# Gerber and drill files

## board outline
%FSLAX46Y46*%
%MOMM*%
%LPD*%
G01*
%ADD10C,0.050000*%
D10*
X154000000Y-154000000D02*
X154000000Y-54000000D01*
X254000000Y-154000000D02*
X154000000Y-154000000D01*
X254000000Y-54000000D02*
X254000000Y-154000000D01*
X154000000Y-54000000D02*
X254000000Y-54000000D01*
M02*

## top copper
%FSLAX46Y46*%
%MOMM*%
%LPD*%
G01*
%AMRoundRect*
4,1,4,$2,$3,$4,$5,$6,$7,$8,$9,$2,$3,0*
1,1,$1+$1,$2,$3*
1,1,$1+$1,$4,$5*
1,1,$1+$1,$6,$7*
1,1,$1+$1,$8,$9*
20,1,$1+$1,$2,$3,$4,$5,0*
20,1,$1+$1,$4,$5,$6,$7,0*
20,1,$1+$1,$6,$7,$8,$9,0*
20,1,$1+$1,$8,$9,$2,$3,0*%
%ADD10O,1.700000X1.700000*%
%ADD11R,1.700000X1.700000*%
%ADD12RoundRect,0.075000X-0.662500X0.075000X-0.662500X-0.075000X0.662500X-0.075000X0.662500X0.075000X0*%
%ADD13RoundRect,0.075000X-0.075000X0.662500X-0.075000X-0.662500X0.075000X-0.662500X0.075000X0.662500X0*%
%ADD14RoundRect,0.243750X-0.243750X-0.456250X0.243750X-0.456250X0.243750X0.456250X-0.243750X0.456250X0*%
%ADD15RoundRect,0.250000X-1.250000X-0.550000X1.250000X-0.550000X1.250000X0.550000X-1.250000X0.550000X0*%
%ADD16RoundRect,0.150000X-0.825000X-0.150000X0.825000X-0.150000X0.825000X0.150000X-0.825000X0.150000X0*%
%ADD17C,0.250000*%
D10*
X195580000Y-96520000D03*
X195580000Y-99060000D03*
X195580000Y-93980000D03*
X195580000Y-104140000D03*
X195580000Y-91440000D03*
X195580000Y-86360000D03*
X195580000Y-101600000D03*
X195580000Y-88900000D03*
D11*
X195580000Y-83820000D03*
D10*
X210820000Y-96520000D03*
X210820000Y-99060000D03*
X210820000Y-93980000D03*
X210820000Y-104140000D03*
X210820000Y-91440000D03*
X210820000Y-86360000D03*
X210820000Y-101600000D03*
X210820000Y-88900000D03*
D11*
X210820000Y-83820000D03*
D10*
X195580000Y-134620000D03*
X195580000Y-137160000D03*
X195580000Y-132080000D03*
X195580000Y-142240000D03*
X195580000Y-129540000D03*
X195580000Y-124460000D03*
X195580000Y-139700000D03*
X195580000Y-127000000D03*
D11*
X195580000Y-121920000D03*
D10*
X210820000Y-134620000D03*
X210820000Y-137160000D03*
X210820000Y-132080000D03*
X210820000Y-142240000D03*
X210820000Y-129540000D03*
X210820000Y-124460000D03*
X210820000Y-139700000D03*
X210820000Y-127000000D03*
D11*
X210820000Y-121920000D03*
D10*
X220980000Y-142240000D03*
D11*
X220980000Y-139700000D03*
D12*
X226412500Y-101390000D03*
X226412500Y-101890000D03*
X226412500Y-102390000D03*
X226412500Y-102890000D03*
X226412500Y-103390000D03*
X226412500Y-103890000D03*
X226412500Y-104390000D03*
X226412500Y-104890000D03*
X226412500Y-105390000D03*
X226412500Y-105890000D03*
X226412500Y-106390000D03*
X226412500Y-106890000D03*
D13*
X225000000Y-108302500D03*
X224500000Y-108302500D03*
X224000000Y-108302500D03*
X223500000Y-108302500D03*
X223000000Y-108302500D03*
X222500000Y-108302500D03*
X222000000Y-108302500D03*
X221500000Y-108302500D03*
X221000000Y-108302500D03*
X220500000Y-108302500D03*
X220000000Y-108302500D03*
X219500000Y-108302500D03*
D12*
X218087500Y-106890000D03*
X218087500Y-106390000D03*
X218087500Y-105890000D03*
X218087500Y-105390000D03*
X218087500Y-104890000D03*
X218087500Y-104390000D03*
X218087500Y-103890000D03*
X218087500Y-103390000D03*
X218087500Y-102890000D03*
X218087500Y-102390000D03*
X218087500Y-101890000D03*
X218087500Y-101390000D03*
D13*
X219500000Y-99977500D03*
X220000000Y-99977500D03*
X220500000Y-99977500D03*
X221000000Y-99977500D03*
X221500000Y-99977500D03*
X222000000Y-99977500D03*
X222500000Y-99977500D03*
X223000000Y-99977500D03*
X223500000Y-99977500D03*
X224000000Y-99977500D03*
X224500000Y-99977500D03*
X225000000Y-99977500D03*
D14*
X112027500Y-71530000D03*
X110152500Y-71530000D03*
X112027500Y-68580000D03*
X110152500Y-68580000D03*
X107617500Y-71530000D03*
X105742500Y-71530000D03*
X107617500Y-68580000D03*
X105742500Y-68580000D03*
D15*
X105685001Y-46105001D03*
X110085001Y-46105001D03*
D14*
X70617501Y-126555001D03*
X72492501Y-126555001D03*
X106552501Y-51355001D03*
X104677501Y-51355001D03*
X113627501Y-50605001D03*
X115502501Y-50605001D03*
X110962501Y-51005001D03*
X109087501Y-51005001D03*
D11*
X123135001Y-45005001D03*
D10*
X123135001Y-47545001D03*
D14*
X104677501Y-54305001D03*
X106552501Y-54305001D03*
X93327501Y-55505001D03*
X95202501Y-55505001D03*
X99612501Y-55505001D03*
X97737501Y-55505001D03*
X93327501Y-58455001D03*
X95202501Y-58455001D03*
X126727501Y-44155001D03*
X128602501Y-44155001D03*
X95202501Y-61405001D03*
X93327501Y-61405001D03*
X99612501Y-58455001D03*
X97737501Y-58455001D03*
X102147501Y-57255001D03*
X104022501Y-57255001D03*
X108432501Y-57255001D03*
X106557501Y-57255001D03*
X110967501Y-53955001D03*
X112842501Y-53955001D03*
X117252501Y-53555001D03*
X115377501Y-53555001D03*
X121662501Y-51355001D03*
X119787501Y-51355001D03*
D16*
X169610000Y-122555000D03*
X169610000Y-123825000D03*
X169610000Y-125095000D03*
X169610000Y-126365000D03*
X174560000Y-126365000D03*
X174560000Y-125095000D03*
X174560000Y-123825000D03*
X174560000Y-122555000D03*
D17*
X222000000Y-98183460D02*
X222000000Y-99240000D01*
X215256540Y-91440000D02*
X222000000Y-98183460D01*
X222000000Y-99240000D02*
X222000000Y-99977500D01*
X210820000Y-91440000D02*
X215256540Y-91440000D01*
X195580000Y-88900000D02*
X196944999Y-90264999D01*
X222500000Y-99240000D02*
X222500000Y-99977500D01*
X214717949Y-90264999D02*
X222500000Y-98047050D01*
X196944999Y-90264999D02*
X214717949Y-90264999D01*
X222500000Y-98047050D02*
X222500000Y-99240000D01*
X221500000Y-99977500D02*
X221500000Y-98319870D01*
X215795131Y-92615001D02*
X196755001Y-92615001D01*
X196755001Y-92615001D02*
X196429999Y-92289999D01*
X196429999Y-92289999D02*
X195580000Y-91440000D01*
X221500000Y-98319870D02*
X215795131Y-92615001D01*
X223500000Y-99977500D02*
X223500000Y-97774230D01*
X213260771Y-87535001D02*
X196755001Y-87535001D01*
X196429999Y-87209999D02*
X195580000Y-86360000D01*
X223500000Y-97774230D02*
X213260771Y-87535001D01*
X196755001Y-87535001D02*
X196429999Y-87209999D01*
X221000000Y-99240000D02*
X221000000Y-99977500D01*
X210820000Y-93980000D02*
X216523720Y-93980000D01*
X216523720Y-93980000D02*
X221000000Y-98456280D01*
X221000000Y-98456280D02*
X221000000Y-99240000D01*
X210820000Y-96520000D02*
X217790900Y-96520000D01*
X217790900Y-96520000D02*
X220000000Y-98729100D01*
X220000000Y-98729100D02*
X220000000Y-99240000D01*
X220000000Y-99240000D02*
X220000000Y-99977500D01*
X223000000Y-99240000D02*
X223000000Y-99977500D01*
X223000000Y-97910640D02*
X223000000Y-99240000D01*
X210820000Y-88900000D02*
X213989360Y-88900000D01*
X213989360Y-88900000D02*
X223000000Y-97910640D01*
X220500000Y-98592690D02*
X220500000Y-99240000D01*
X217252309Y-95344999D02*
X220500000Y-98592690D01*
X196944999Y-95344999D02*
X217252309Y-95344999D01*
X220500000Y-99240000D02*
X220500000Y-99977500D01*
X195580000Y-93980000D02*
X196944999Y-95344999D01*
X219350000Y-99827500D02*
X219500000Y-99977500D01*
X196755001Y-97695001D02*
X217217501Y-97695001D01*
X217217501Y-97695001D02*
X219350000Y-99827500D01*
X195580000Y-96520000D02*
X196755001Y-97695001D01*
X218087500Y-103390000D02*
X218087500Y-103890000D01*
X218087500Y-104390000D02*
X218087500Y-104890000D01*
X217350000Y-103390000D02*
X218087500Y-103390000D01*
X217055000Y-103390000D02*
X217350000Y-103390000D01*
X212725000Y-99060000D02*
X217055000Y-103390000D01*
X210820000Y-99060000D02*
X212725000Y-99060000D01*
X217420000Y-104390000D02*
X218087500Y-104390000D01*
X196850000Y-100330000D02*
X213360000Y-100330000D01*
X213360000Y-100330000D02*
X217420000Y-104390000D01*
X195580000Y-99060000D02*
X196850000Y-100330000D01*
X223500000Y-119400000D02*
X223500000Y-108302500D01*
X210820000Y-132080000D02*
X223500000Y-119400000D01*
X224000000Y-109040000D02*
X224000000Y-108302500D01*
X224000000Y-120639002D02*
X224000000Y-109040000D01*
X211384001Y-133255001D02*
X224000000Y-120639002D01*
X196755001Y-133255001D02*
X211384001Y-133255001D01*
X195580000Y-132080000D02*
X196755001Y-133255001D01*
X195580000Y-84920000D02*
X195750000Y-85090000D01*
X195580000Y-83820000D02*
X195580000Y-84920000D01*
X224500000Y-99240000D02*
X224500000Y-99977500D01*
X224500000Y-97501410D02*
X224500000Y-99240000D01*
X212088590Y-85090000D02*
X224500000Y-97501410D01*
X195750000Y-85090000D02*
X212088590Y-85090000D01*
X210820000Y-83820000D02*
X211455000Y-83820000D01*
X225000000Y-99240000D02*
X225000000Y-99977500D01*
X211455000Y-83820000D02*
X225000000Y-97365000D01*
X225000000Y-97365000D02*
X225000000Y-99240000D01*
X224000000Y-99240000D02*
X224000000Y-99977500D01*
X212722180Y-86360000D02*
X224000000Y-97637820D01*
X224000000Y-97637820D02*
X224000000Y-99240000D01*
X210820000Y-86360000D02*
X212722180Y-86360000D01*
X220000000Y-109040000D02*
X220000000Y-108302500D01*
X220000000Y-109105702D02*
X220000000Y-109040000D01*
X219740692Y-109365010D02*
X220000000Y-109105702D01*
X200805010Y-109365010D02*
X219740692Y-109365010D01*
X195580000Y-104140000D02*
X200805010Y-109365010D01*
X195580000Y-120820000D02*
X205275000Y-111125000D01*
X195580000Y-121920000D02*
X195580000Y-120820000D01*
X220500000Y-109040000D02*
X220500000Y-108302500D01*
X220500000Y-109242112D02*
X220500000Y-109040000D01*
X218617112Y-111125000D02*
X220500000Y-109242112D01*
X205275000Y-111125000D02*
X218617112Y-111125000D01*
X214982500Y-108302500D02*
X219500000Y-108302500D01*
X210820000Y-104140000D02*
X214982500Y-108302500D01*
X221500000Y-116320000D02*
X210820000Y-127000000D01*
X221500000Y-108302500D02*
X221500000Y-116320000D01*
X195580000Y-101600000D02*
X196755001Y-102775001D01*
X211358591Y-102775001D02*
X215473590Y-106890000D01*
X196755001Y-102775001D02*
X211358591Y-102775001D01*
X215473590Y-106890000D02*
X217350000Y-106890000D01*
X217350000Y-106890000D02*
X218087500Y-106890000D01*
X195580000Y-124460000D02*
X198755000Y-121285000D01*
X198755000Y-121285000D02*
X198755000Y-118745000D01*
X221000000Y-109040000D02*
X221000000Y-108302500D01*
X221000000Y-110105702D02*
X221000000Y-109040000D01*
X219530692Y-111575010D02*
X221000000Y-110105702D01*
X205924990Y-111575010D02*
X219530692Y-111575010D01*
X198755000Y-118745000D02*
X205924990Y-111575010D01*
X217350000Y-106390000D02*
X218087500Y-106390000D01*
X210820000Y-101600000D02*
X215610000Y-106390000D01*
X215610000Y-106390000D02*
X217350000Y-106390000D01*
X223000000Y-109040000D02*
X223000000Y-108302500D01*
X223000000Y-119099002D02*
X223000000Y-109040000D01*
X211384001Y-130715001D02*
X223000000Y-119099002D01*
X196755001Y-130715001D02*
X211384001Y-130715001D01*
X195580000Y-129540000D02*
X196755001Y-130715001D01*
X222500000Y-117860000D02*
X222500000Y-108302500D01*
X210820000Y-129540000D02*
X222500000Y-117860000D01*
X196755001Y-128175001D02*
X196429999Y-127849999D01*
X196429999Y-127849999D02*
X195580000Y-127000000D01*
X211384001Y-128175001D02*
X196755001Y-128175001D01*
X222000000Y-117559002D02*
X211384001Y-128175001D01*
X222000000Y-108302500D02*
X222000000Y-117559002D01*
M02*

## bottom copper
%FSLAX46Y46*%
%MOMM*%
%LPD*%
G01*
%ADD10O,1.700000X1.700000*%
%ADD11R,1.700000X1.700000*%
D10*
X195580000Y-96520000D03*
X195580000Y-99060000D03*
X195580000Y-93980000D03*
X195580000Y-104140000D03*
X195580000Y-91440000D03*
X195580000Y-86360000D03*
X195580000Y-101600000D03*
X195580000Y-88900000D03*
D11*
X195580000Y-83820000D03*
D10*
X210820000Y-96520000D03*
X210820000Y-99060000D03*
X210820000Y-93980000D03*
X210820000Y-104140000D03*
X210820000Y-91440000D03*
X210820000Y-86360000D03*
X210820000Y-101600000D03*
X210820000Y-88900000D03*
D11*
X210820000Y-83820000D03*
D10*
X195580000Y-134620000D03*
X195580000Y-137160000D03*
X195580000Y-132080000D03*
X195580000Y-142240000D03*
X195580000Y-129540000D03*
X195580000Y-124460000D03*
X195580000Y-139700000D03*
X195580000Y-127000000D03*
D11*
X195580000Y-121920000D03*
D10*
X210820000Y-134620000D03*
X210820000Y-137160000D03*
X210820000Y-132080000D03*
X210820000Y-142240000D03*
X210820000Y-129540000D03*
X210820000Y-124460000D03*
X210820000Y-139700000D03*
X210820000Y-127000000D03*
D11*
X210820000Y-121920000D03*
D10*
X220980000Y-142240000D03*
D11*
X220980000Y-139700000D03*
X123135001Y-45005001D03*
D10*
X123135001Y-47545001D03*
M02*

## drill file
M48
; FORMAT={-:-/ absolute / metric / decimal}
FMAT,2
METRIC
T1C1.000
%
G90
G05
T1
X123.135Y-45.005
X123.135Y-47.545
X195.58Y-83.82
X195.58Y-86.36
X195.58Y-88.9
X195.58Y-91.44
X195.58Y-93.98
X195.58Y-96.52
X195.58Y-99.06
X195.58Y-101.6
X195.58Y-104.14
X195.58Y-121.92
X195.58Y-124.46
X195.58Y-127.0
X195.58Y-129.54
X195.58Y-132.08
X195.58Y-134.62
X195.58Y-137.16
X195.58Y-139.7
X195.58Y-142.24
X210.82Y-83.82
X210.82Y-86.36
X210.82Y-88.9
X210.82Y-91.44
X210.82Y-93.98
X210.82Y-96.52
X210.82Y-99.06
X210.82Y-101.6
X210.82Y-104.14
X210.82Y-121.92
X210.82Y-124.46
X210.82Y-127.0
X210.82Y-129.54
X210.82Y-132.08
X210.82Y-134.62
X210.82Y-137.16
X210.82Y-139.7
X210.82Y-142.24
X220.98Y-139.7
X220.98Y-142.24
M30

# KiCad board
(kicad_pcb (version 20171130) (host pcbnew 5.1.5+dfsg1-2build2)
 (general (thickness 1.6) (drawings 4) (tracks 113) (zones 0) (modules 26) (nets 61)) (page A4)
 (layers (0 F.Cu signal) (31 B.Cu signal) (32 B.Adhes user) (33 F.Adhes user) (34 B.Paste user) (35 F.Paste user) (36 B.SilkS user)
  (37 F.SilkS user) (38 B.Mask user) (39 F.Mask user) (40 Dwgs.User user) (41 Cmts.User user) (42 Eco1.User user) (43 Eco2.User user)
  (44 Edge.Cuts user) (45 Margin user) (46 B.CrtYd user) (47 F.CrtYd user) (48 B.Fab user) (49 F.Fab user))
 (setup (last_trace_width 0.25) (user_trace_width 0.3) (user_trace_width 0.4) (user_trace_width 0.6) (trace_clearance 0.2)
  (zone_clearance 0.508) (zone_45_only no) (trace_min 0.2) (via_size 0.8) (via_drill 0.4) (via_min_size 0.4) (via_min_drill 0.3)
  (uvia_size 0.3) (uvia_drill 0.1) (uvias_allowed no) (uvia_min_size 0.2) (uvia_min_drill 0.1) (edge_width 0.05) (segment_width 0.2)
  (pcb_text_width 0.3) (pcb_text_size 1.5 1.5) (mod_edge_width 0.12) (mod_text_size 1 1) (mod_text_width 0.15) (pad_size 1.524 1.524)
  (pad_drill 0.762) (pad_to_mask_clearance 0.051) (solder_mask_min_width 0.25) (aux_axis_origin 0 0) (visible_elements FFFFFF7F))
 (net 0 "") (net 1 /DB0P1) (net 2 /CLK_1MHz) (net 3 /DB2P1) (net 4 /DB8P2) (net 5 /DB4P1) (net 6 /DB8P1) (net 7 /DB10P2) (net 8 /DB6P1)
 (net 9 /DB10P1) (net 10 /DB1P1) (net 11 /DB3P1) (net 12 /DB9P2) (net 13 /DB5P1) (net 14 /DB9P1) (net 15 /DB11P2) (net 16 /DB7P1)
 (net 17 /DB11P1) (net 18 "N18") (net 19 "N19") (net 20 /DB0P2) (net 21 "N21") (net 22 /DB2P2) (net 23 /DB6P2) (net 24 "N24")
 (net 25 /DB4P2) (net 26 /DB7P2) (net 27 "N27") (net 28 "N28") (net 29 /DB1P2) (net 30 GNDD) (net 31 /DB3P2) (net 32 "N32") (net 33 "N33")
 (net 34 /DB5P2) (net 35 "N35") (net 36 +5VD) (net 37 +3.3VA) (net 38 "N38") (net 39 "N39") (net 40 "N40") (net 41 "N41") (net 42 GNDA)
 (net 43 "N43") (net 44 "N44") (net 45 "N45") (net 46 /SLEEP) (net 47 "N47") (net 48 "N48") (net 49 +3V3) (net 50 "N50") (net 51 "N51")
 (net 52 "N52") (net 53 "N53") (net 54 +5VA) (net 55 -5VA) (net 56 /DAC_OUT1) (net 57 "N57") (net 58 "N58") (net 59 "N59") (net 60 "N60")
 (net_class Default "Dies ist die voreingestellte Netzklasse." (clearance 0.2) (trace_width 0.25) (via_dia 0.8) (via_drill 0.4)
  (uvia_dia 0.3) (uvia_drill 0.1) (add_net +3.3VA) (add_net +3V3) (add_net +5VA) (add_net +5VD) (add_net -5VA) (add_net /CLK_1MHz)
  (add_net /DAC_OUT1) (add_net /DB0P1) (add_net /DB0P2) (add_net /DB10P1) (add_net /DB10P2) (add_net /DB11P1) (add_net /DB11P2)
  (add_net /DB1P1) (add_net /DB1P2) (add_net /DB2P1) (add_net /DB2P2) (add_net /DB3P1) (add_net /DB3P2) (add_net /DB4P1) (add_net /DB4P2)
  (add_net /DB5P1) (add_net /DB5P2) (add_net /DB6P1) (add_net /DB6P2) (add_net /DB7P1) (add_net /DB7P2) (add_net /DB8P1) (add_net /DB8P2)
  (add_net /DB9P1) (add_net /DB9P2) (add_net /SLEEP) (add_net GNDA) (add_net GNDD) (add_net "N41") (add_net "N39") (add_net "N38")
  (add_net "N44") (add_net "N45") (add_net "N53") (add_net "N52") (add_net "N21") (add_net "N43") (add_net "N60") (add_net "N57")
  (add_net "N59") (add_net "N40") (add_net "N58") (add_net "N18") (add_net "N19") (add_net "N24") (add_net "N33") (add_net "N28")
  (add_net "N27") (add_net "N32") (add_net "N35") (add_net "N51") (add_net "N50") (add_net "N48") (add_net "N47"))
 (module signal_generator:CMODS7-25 (layer F.Cu) (at 195.58 83.82)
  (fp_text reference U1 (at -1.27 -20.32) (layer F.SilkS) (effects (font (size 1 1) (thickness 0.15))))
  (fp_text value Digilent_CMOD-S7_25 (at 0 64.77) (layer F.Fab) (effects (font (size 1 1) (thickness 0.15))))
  (pad 6 thru_hole oval (at 0 12.7) (size 1.7 1.7) (drill 1) (layers *.Cu *.Mask) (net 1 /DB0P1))
  (pad 7 thru_hole oval (at 0 15.24) (size 1.7 1.7) (drill 1) (layers *.Cu *.Mask) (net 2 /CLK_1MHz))
  (pad 5 thru_hole oval (at 0 10.16) (size 1.7 1.7) (drill 1) (layers *.Cu *.Mask) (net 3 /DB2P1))
  (pad 9 thru_hole oval (at 0 20.32) (size 1.7 1.7) (drill 1) (layers *.Cu *.Mask) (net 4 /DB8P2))
  (pad 4 thru_hole oval (at 0 7.62) (size 1.7 1.7) (drill 1) (layers *.Cu *.Mask) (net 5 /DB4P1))
  (pad 2 thru_hole oval (at 0 2.54) (size 1.7 1.7) (drill 1) (layers *.Cu *.Mask) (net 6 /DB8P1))
  (pad 8 thru_hole oval (at 0 17.78) (size 1.7 1.7) (drill 1) (layers *.Cu *.Mask) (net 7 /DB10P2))
  (pad 3 thru_hole oval (at 0 5.08) (size 1.7 1.7) (drill 1) (layers *.Cu *.Mask) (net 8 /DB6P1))
  (pad 1 thru_hole rect (at 0 0) (size 1.7 1.7) (drill 1) (layers *.Cu *.Mask) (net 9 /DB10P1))
  (pad 43 thru_hole oval (at 15.24 12.7) (size 1.7 1.7) (drill 1) (layers *.Cu *.Mask) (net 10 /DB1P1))
  (pad 42 thru_hole oval (at 15.24 15.24) (size 1.7 1.7) (drill 1) (layers *.Cu *.Mask) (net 2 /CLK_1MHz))
  (pad 44 thru_hole oval (at 15.24 10.16) (size 1.7 1.7) (drill 1) (layers *.Cu *.Mask) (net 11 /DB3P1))
  (pad 40 thru_hole oval (at 15.24 20.32) (size 1.7 1.7) (drill 1) (layers *.Cu *.Mask) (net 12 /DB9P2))
  (pad 45 thru_hole oval (at 15.24 7.62) (size 1.7 1.7) (drill 1) (layers *.Cu *.Mask) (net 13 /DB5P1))
  (pad 47 thru_hole oval (at 15.24 2.54) (size 1.7 1.7) (drill 1) (layers *.Cu *.Mask) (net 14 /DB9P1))
  (pad 41 thru_hole oval (at 15.24 17.78) (size 1.7 1.7) (drill 1) (layers *.Cu *.Mask) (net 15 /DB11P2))
  (pad 46 thru_hole oval (at 15.24 5.08) (size 1.7 1.7) (drill 1) (layers *.Cu *.Mask) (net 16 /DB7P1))
  (pad 48 thru_hole rect (at 15.24 0) (size 1.7 1.7) (drill 1) (layers *.Cu *.Mask) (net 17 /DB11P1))
  (pad 21 thru_hole oval (at 0 50.8) (size 1.7 1.7) (drill 1) (layers *.Cu *.Mask) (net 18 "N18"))
  (pad 22 thru_hole oval (at 0 53.34) (size 1.7 1.7) (drill 1) (layers *.Cu *.Mask) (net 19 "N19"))
  (pad 20 thru_hole oval (at 0 48.26) (size 1.7 1.7) (drill 1) (layers *.Cu *.Mask) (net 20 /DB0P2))
  (pad 24 thru_hole oval (at 0 58.42) (size 1.7 1.7) (drill 1) (layers *.Cu *.Mask) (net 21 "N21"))
  (pad 19 thru_hole oval (at 0 45.72) (size 1.7 1.7) (drill 1) (layers *.Cu *.Mask) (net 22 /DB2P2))
  (pad 17 thru_hole oval (at 0 40.64) (size 1.7 1.7) (drill 1) (layers *.Cu *.Mask) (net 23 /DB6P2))
  (pad 23 thru_hole oval (at 0 55.88) (size 1.7 1.7) (drill 1) (layers *.Cu *.Mask) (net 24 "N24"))
  (pad 18 thru_hole oval (at 0 43.18) (size 1.7 1.7) (drill 1) (layers *.Cu *.Mask) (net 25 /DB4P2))
  (pad 16 thru_hole rect (at 0 38.1) (size 1.7 1.7) (drill 1) (layers *.Cu *.Mask) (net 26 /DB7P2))
  (pad 28 thru_hole oval (at 15.24 50.8) (size 1.7 1.7) (drill 1) (layers *.Cu *.Mask) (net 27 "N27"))
  (pad 27 thru_hole oval (at 15.24 53.34) (size 1.7 1.7) (drill 1) (layers *.Cu *.Mask) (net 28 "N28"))
  (pad 29 thru_hole oval (at 15.24 48.26) (size 1.7 1.7) (drill 1) (layers *.Cu *.Mask) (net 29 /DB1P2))
  (pad 25 thru_hole oval (at 15.24 58.42) (size 1.7 1.7) (drill 1) (layers *.Cu *.Mask) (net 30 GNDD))
  (pad 30 thru_hole oval (at 15.24 45.72) (size 1.7 1.7) (drill 1) (layers *.Cu *.Mask) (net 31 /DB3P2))
  (pad 32 thru_hole oval (at 15.24 40.64) (size 1.7 1.7) (drill 1) (layers *.Cu *.Mask) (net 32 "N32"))
  (pad 26 thru_hole oval (at 15.24 55.88) (size 1.7 1.7) (drill 1) (layers *.Cu *.Mask) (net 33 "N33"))
  (pad 31 thru_hole oval (at 15.24 43.18) (size 1.7 1.7) (drill 1) (layers *.Cu *.Mask) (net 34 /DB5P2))
  (pad 33 thru_hole rect (at 15.24 38.1) (size 1.7 1.7) (drill 1) (layers *.Cu *.Mask) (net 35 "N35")))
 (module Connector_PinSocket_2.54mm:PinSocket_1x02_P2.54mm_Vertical (layer F.Cu) (at 220.98 139.7)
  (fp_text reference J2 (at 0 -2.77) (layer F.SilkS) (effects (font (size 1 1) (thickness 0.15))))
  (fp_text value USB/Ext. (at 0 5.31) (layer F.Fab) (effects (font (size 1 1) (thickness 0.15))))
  (pad 2 thru_hole oval (at 0 2.54) (size 1.7 1.7) (drill 1) (layers *.Cu *.Mask) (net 21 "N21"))
  (pad 1 thru_hole rect (at 0 0) (size 1.7 1.7) (drill 1) (layers *.Cu *.Mask) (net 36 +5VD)))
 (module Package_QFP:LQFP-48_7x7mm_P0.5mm (layer F.Cu) (at 222.25 104.14 270)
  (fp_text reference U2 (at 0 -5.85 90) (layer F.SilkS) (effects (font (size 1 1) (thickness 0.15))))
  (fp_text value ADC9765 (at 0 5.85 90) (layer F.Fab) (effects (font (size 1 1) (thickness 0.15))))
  (pad 48 smd roundrect (at -2.75 -4.1625 270) (size 0.3 1.475) (layers F.Cu F.Paste F.Mask) (roundrect_rratio 0.25) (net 36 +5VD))
  (pad 47 smd roundrect (at -2.25 -4.1625 270) (size 0.3 1.475) (layers F.Cu F.Paste F.Mask) (roundrect_rratio 0.25) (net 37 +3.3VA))
  (pad 46 smd roundrect (at -1.75 -4.1625 270) (size 0.3 1.475) (layers F.Cu F.Paste F.Mask) (roundrect_rratio 0.25) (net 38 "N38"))
  (pad 45 smd roundrect (at -1.25 -4.1625 270) (size 0.3 1.475) (layers F.Cu F.Paste F.Mask) (roundrect_rratio 0.25) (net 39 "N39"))
  (pad 44 smd roundrect (at -0.75 -4.1625 270) (size 0.3 1.475) (layers F.Cu F.Paste F.Mask) (roundrect_rratio 0.25) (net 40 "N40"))
  (pad 43 smd roundrect (at -0.25 -4.1625 270) (size 0.3 1.475) (layers F.Cu F.Paste F.Mask) (roundrect_rratio 0.25) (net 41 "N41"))
  (pad 42 smd roundrect (at 0.25 -4.1625 270) (size 0.3 1.475) (layers F.Cu F.Paste F.Mask) (roundrect_rratio 0.25) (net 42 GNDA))
  (pad 41 smd roundrect (at 0.75 -4.1625 270) (size 0.3 1.475) (layers F.Cu F.Paste F.Mask) (roundrect_rratio 0.25) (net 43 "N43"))
  (pad 40 smd roundrect (at 1.25 -4.1625 270) (size 0.3 1.475) (layers F.Cu F.Paste F.Mask) (roundrect_rratio 0.25) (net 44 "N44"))
  (pad 39 smd roundrect (at 1.75 -4.1625 270) (size 0.3 1.475) (layers F.Cu F.Paste F.Mask) (roundrect_rratio 0.25) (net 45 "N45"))
  (pad 38 smd roundrect (at 2.25 -4.1625 270) (size 0.3 1.475) (layers F.Cu F.Paste F.Mask) (roundrect_rratio 0.25) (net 42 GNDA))
  (pad 37 smd roundrect (at 2.75 -4.1625 270) (size 0.3 1.475) (layers F.Cu F.Paste F.Mask) (roundrect_rratio 0.25) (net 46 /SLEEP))
  (pad 36 smd roundrect (at 4.1625 -2.75 270) (size 1.475 0.3) (layers F.Cu F.Paste F.Mask) (roundrect_rratio 0.25) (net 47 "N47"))
  (pad 35 smd roundrect (at 4.1625 -2.25 270) (size 1.475 0.3) (layers F.Cu F.Paste F.Mask) (roundrect_rratio 0.25) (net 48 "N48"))
  (pad 34 smd roundrect (at 4.1625 -1.75 270) (size 1.475 0.3) (layers F.Cu F.Paste F.Mask) (roundrect_rratio 0.25) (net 20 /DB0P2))
  (pad 33 smd roundrect (at 4.1625 -1.25 270) (size 1.475 0.3) (layers F.Cu F.Paste F.Mask) (roundrect_rratio 0.25) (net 29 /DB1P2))
  (pad 32 smd roundrect (at 4.1625 -0.75 270) (size 1.475 0.3) (layers F.Cu F.Paste F.Mask) (roundrect_rratio 0.25) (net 22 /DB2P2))
  (pad 31 smd roundrect (at 4.1625 -0.25 270) (size 1.475 0.3) (layers F.Cu F.Paste F.Mask) (roundrect_rratio 0.25) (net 31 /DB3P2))
  (pad 30 smd roundrect (at 4.1625 0.25 270) (size 1.475 0.3) (layers F.Cu F.Paste F.Mask) (roundrect_rratio 0.25) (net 25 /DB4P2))
  (pad 29 smd roundrect (at 4.1625 0.75 270) (size 1.475 0.3) (layers F.Cu F.Paste F.Mask) (roundrect_rratio 0.25) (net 34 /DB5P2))
  (pad 28 smd roundrect (at 4.1625 1.25 270) (size 1.475 0.3) (layers F.Cu F.Paste F.Mask) (roundrect_rratio 0.25) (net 23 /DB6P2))
  (pad 27 smd roundrect (at 4.1625 1.75 270) (size 1.475 0.3) (layers F.Cu F.Paste F.Mask) (roundrect_rratio 0.25) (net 26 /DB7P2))
  (pad 26 smd roundrect (at 4.1625 2.25 270) (size 1.475 0.3) (layers F.Cu F.Paste F.Mask) (roundrect_rratio 0.25) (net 4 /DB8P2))
  (pad 25 smd roundrect (at 4.1625 2.75 270) (size 1.475 0.3) (layers F.Cu F.Paste F.Mask) (roundrect_rratio 0.25) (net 12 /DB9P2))
  (pad 24 smd roundrect (at 2.75 4.1625 270) (size 0.3 1.475) (layers F.Cu F.Paste F.Mask) (roundrect_rratio 0.25) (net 7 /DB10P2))
  (pad 23 smd roundrect (at 2.25 4.1625 270) (size 0.3 1.475) (layers F.Cu F.Paste F.Mask) (roundrect_rratio 0.25) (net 15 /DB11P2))
  (pad 22 smd roundrect (at 1.75 4.1625 270) (size 0.3 1.475) (layers F.Cu F.Paste F.Mask) (roundrect_rratio 0.25) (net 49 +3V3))
  (pad 21 smd roundrect (at 1.25 4.1625 270) (size 0.3 1.475) (layers F.Cu F.Paste F.Mask) (roundrect_rratio 0.25) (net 30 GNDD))
  (pad 20 smd roundrect (at 0.75 4.1625 270) (size 0.3 1.475) (layers F.Cu F.Paste F.Mask) (roundrect_rratio 0.25) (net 2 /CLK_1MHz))
  (pad 19 smd roundrect (at 0.25 4.1625 270) (size 0.3 1.475) (layers F.Cu F.Paste F.Mask) (roundrect_rratio 0.25) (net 2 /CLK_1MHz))
  (pad 18 smd roundrect (at -0.25 4.1625 270) (size 0.3 1.475) (layers F.Cu F.Paste F.Mask) (roundrect_rratio 0.25) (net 2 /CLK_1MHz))
  (pad 17 smd roundrect (at -0.75 4.1625 270) (size 0.3 1.475) (layers F.Cu F.Paste F.Mask) (roundrect_rratio 0.25) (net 2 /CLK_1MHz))
  (pad 16 smd roundrect (at -1.25 4.1625 270) (size 0.3 1.475) (layers F.Cu F.Paste F.Mask) (roundrect_rratio 0.25) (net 49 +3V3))
  (pad 15 smd roundrect (at -1.75 4.1625 270) (size 0.3 1.475) (layers F.Cu F.Paste F.Mask) (roundrect_rratio 0.25) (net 30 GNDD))
  (pad 14 smd roundrect (at -2.25 4.1625 270) (size 0.3 1.475) (layers F.Cu F.Paste F.Mask) (roundrect_rratio 0.25) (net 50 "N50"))
  (pad 13 smd roundrect (at -2.75 4.1625 270) (size 0.3 1.475) (layers F.Cu F.Paste F.Mask) (roundrect_rratio 0.25) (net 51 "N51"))
  (pad 12 smd roundrect (at -4.1625 2.75 270) (size 1.475 0.3) (layers F.Cu F.Paste F.Mask) (roundrect_rratio 0.25) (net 1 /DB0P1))
  (pad 11 smd roundrect (at -4.1625 2.25 270) (size 1.475 0.3) (layers F.Cu F.Paste F.Mask) (roundrect_rratio 0.25) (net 10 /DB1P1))
  (pad 10 smd roundrect (at -4.1625 1.75 270) (size 1.475 0.3) (layers F.Cu F.Paste F.Mask) (roundrect_rratio 0.25) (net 3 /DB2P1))
  (pad 9 smd roundrect (at -4.1625 1.25 270) (size 1.475 0.3) (layers F.Cu F.Paste F.Mask) (roundrect_rratio 0.25) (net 11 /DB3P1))
  (pad 8 smd roundrect (at -4.1625 0.75 270) (size 1.475 0.3) (layers F.Cu F.Paste F.Mask) (roundrect_rratio 0.25) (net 5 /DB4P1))
  (pad 7 smd roundrect (at -4.1625 0.25 270) (size 1.475 0.3) (layers F.Cu F.Paste F.Mask) (roundrect_rratio 0.25) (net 13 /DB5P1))
  (pad 6 smd roundrect (at -4.1625 -0.25 270) (size 1.475 0.3) (layers F.Cu F.Paste F.Mask) (roundrect_rratio 0.25) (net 8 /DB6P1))
  (pad 5 smd roundrect (at -4.1625 -0.75 270) (size 1.475 0.3) (layers F.Cu F.Paste F.Mask) (roundrect_rratio 0.25) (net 16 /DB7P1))
  (pad 4 smd roundrect (at -4.1625 -1.25 270) (size 1.475 0.3) (layers F.Cu F.Paste F.Mask) (roundrect_rratio 0.25) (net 6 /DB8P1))
  (pad 3 smd roundrect (at -4.1625 -1.75 270) (size 1.475 0.3) (layers F.Cu F.Paste F.Mask) (roundrect_rratio 0.25) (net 14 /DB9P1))
  (pad 2 smd roundrect (at -4.1625 -2.25 270) (size 1.475 0.3) (layers F.Cu F.Paste F.Mask) (roundrect_rratio 0.25) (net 9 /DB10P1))
  (pad 1 smd roundrect (at -4.1625 -2.75 270) (size 1.475 0.3) (layers F.Cu F.Paste F.Mask) (roundrect_rratio 0.25) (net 17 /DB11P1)))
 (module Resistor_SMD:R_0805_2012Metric (layer F.Cu) (at 111.09 71.53)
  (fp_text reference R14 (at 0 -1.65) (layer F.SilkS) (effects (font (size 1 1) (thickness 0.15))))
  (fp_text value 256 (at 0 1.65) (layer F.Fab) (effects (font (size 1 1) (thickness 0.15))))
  (pad 2 smd roundrect (at 0.9375 0) (size 0.975 1.4) (layers F.Cu F.Paste F.Mask) (roundrect_rratio 0.25) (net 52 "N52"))
  (pad 1 smd roundrect (at -0.9375 0) (size 0.975 1.4) (layers F.Cu F.Paste F.Mask) (roundrect_rratio 0.25) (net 40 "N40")))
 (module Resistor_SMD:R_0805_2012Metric (layer F.Cu) (at 111.09 68.58)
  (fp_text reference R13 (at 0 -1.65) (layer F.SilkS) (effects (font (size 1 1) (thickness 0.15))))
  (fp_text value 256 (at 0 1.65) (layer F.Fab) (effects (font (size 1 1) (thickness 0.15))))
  (pad 2 smd roundrect (at 0.9375 0) (size 0.975 1.4) (layers F.Cu F.Paste F.Mask) (roundrect_rratio 0.25) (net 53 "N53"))
  (pad 1 smd roundrect (at -0.9375 0) (size 0.975 1.4) (layers F.Cu F.Paste F.Mask) (roundrect_rratio 0.25) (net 43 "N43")))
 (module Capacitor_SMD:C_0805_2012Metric (layer F.Cu) (at 106.68 71.53)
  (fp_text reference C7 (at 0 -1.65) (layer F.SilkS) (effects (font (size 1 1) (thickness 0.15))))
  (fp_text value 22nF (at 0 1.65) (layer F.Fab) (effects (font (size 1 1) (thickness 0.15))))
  (pad 2 smd roundrect (at 0.9375 0) (size 0.975 1.4) (layers F.Cu F.Paste F.Mask) (roundrect_rratio 0.25) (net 42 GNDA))
  (pad 1 smd roundrect (at -0.9375 0) (size 0.975 1.4) (layers F.Cu F.Paste F.Mask) (roundrect_rratio 0.25) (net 52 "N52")))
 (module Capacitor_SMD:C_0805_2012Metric (layer F.Cu) (at 106.68 68.58)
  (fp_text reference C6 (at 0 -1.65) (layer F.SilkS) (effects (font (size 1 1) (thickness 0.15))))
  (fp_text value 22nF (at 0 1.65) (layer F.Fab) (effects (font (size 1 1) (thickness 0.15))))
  (pad 2 smd roundrect (at 0.9375 0) (size 0.975 1.4) (layers F.Cu F.Paste F.Mask) (roundrect_rratio 0.25) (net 42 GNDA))
  (pad 1 smd roundrect (at -0.9375 0) (size 0.975 1.4) (layers F.Cu F.Paste F.Mask) (roundrect_rratio 0.25) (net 53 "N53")))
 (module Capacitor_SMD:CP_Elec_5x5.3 (layer F.Cu) (at 107.885001 46.105001)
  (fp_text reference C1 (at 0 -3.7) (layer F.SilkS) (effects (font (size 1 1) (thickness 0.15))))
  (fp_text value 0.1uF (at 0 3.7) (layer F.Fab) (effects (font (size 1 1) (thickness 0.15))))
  (pad 1 smd roundrect (at -2.2 0) (size 3 1.6) (layers F.Cu F.Paste F.Mask) (roundrect_rratio 0.15625) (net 41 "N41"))
  (pad 2 smd roundrect (at 2.2 0) (size 3 1.6) (layers F.Cu F.Paste F.Mask) (roundrect_rratio 0.15625) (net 42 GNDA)))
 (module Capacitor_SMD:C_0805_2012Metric (layer F.Cu) (at 71.555001 126.555001)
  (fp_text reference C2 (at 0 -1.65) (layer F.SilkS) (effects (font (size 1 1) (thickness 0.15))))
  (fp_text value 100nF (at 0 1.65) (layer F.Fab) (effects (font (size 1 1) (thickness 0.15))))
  (pad 1 smd roundrect (at -0.9375 0) (size 0.975 1.4) (layers F.Cu F.Paste F.Mask) (roundrect_rratio 0.25) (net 39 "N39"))
  (pad 2 smd roundrect (at 0.9375 0) (size 0.975 1.4) (layers F.Cu F.Paste F.Mask) (roundrect_rratio 0.25) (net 38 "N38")))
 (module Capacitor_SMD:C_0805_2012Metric (layer F.Cu) (at 105.615001 51.355001)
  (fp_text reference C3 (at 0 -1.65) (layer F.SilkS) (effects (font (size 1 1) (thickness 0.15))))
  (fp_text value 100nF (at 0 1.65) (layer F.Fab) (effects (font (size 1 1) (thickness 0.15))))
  (pad 2 smd roundrect (at 0.9375 0) (size 0.975 1.4) (layers F.Cu F.Paste F.Mask) (roundrect_rratio 0.25) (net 45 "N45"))
  (pad 1 smd roundrect (at -0.9375 0) (size 0.975 1.4) (layers F.Cu F.Paste F.Mask) (roundrect_rratio 0.25) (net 44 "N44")))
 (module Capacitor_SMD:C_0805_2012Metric (layer F.Cu) (at 114.565001 50.605001)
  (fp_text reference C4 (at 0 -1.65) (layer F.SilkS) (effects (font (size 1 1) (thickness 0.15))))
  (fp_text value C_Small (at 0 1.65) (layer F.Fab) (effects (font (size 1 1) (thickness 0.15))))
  (pad 1 smd roundrect (at -0.9375 0) (size 0.975 1.4) (layers F.Cu F.Paste F.Mask) (roundrect_rratio 0.25) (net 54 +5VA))
  (pad 2 smd roundrect (at 0.9375 0) (size 0.975 1.4) (layers F.Cu F.Paste F.Mask) (roundrect_rratio 0.25) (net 42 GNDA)))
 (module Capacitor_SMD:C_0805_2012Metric (layer F.Cu) (at 110.025001 51.005001)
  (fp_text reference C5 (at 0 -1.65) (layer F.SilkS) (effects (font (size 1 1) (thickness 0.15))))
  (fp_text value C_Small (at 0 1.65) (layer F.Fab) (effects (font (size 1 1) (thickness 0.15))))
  (pad 2 smd roundrect (at 0.9375 0) (size 0.975 1.4) (layers F.Cu F.Paste F.Mask) (roundrect_rratio 0.25) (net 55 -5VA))
  (pad 1 smd roundrect (at -0.9375 0) (size 0.975 1.4) (layers F.Cu F.Paste F.Mask) (roundrect_rratio 0.25) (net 42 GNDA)))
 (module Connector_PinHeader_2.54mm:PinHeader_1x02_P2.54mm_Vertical (layer F.Cu) (at 123.135001 45.005001)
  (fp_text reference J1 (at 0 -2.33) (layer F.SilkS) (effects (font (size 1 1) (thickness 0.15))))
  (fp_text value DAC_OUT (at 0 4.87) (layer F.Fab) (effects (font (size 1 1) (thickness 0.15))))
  (pad 1 thru_hole rect (at 0 0) (size 1.7 1.7) (drill 1) (layers *.Cu *.Mask) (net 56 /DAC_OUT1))
  (pad 2 thru_hole oval (at 0 2.54) (size 1.7 1.7) (drill 1) (layers *.Cu *.Mask) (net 56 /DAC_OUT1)))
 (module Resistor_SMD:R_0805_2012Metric (layer F.Cu) (at 105.615001 54.305001)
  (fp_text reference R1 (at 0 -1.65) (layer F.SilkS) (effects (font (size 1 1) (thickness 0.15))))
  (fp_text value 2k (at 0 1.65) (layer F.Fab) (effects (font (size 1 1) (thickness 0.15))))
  (pad 1 smd roundrect (at -0.9375 0) (size 0.975 1.4) (layers F.Cu F.Paste F.Mask) (roundrect_rratio 0.25) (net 43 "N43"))
  (pad 2 smd roundrect (at 0.9375 0) (size 0.975 1.4) (layers F.Cu F.Paste F.Mask) (roundrect_rratio 0.25) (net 42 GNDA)))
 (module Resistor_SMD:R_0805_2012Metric (layer F.Cu) (at 94.265001 55.505001)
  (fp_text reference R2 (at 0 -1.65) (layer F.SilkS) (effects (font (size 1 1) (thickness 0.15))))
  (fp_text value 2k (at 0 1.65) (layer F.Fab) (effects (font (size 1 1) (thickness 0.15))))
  (pad 1 smd roundrect (at -0.9375 0) (size 0.975 1.4) (layers F.Cu F.Paste F.Mask) (roundrect_rratio 0.25) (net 40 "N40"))
  (pad 2 smd roundrect (at 0.9375 0) (size 0.975 1.4) (layers F.Cu F.Paste F.Mask) (roundrect_rratio 0.25) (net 42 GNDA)))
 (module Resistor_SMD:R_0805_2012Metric (layer F.Cu) (at 98.675001 55.505001)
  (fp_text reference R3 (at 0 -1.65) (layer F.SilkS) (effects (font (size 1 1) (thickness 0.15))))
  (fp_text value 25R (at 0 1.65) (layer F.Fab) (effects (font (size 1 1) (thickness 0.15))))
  (pad 2 smd roundrect (at 0.9375 0) (size 0.975 1.4) (layers F.Cu F.Paste F.Mask) (roundrect_rratio 0.25) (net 42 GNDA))
  (pad 1 smd roundrect (at -0.9375 0) (size 0.975 1.4) (layers F.Cu F.Paste F.Mask) (roundrect_rratio 0.25) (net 39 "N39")))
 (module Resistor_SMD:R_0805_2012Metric (layer F.Cu) (at 94.265001 58.455001)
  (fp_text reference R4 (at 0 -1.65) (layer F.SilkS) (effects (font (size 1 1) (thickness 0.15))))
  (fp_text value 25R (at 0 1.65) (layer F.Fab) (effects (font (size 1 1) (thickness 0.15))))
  (pad 1 smd roundrect (at -0.9375 0) (size 0.975 1.4) (layers F.Cu F.Paste F.Mask) (roundrect_rratio 0.25) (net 44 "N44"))
  (pad 2 smd roundrect (at 0.9375 0) (size 0.975 1.4) (layers F.Cu F.Paste F.Mask) (roundrect_rratio 0.25) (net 42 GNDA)))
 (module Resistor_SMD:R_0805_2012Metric (layer F.Cu) (at 127.665001 44.155001)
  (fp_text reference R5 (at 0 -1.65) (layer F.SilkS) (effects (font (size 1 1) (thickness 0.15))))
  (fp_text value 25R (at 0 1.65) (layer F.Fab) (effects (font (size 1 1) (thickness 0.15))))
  (pad 1 smd roundrect (at -0.9375 0) (size 0.975 1.4) (layers F.Cu F.Paste F.Mask) (roundrect_rratio 0.25) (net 38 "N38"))
  (pad 2 smd roundrect (at 0.9375 0) (size 0.975 1.4) (layers F.Cu F.Paste F.Mask) (roundrect_rratio 0.25) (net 42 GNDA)))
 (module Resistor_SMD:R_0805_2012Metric (layer F.Cu) (at 94.265001 61.405001)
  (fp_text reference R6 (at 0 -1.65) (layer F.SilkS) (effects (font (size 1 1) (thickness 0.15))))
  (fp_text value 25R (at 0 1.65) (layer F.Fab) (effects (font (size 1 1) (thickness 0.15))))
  (pad 2 smd roundrect (at 0.9375 0) (size 0.975 1.4) (layers F.Cu F.Paste F.Mask) (roundrect_rratio 0.25) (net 42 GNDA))
  (pad 1 smd roundrect (at -0.9375 0) (size 0.975 1.4) (layers F.Cu F.Paste F.Mask) (roundrect_rratio 0.25) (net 45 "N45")))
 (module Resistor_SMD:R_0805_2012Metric (layer F.Cu) (at 98.675001 58.455001)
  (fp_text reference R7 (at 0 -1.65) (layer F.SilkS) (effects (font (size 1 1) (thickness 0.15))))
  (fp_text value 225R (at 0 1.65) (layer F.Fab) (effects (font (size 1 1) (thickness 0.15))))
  (pad 2 smd roundrect (at 0.9375 0) (size 0.975 1.4) (layers F.Cu F.Paste F.Mask) (roundrect_rratio 0.25) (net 38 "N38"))
  (pad 1 smd roundrect (at -0.9375 0) (size 0.975 1.4) (layers F.Cu F.Paste F.Mask) (roundrect_rratio 0.25) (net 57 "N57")))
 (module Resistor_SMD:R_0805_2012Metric (layer F.Cu) (at 103.085001 57.255001)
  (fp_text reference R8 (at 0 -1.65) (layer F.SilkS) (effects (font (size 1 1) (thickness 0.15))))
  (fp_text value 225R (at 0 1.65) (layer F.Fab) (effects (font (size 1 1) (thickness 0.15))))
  (pad 1 smd roundrect (at -0.9375 0) (size 0.975 1.4) (layers F.Cu F.Paste F.Mask) (roundrect_rratio 0.25) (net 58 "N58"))
  (pad 2 smd roundrect (at 0.9375 0) (size 0.975 1.4) (layers F.Cu F.Paste F.Mask) (roundrect_rratio 0.25) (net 39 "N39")))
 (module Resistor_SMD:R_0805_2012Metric (layer F.Cu) (at 107.495001 57.255001)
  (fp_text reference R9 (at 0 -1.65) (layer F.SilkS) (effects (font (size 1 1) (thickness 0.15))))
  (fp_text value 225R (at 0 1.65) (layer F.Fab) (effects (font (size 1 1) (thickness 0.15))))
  (pad 2 smd roundrect (at 0.9375 0) (size 0.975 1.4) (layers F.Cu F.Paste F.Mask) (roundrect_rratio 0.25) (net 45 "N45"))
  (pad 1 smd roundrect (at -0.9375 0) (size 0.975 1.4) (layers F.Cu F.Paste F.Mask) (roundrect_rratio 0.25) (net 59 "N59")))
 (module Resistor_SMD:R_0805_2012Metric (layer F.Cu) (at 111.905001 53.955001)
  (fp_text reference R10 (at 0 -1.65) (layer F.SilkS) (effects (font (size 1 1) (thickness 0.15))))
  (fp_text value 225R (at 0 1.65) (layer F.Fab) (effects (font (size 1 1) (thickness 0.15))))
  (pad 1 smd roundrect (at -0.9375 0) (size 0.975 1.4) (layers F.Cu F.Paste F.Mask) (roundrect_rratio 0.25) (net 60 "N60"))
  (pad 2 smd roundrect (at 0.9375 0) (size 0.975 1.4) (layers F.Cu F.Paste F.Mask) (roundrect_rratio 0.25) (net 44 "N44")))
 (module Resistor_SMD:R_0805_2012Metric (layer F.Cu) (at 116.315001 53.555001)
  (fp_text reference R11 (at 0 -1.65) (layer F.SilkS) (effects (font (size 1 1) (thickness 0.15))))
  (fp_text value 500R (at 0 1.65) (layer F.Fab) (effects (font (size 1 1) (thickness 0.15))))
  (pad 2 smd roundrect (at 0.9375 0) (size 0.975 1.4) (layers F.Cu F.Paste F.Mask) (roundrect_rratio 0.25) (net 57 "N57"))
  (pad 1 smd roundrect (at -0.9375 0) (size 0.975 1.4) (layers F.Cu F.Paste F.Mask) (roundrect_rratio 0.25) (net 56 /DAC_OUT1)))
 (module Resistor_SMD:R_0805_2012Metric (layer F.Cu) (at 120.725001 51.355001)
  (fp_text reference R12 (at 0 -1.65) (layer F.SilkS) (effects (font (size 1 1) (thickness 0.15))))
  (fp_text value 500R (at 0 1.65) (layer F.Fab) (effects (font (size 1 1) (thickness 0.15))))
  (pad 2 smd roundrect (at 0.9375 0) (size 0.975 1.4) (layers F.Cu F.Paste F.Mask) (roundrect_rratio 0.25) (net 59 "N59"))
  (pad 1 smd roundrect (at -0.9375 0) (size 0.975 1.4) (layers F.Cu F.Paste F.Mask) (roundrect_rratio 0.25) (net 56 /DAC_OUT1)))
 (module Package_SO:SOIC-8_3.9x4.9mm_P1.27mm (layer F.Cu) (at 172.085 124.46)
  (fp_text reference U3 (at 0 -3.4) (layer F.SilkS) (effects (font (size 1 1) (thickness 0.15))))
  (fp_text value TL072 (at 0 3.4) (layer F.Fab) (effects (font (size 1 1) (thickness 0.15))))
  (pad 1 smd roundrect (at -2.475 -1.905) (size 1.95 0.6) (layers F.Cu F.Paste F.Mask) (roundrect_rratio 0.25) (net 56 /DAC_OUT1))
  (pad 2 smd roundrect (at -2.475 -0.635) (size 1.95 0.6) (layers F.Cu F.Paste F.Mask) (roundrect_rratio 0.25) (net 57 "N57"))
  (pad 3 smd roundrect (at -2.475 0.635) (size 1.95 0.6) (layers F.Cu F.Paste F.Mask) (roundrect_rratio 0.25) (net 58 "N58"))
  (pad 4 smd roundrect (at -2.475 1.905) (size 1.95 0.6) (layers F.Cu F.Paste F.Mask) (roundrect_rratio 0.25) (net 55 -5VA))
  (pad 5 smd roundrect (at 2.475 1.905) (size 1.95 0.6) (layers F.Cu F.Paste F.Mask) (roundrect_rratio 0.25) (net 60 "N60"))
  (pad 6 smd roundrect (at 2.475 0.635) (size 1.95 0.6) (layers F.Cu F.Paste F.Mask) (roundrect_rratio 0.25) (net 59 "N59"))
  (pad 7 smd roundrect (at 2.475 -0.635) (size 1.95 0.6) (layers F.Cu F.Paste F.Mask) (roundrect_rratio 0.25) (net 56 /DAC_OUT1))
  (pad 8 smd roundrect (at 2.475 -1.905) (size 1.95 0.6) (layers F.Cu F.Paste F.Mask) (roundrect_rratio 0.25) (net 54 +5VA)))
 (gr_line (start 154 154) (end 154 54) (layer Edge.Cuts) (width 0.05))
 (gr_line (start 254 154) (end 154 154) (layer Edge.Cuts) (width 0.05))
 (gr_line (start 254 54) (end 254 154) (layer Edge.Cuts) (width 0.05))
 (gr_line (start 154 54) (end 254 54) (layer Edge.Cuts) (width 0.05))
 (segment (start 222 98.18346) (end 222 99.24) (width 0.25) (layer F.Cu) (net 13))
 (segment (start 215.25654 91.44) (end 222 98.18346) (width 0.25) (layer F.Cu) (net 13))
 (segment (start 222 99.24) (end 222 99.9775) (width 0.25) (layer F.Cu) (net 13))
 (segment (start 210.82 91.44) (end 215.25654 91.44) (width 0.25) (layer F.Cu) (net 13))
 (segment (start 195.58 88.9) (end 196.944999 90.264999) (width 0.25) (layer F.Cu) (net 8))
 (segment (start 222.5 99.24) (end 222.5 99.9775) (width 0.25) (layer F.Cu) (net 8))
 (segment (start 214.717949 90.264999) (end 222.5 98.04705) (width 0.25) (layer F.Cu) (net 8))
 (segment (start 196.944999 90.264999) (end 214.717949 90.264999) (width 0.25) (layer F.Cu) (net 8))
 (segment (start 222.5 98.04705) (end 222.5 99.24) (width 0.25) (layer F.Cu) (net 8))
 (segment (start 221.5 99.9775) (end 221.5 98.31987) (width 0.25) (layer F.Cu) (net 5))
 (segment (start 215.795131 92.615001) (end 196.755001 92.615001) (width 0.25) (layer F.Cu) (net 5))
 (segment (start 196.755001 92.615001) (end 196.429999 92.289999) (width 0.25) (layer F.Cu) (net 5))
 (segment (start 196.429999 92.289999) (end 195.58 91.44) (width 0.25) (layer F.Cu) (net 5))
 (segment (start 221.5 98.31987) (end 215.795131 92.615001) (width 0.25) (layer F.Cu) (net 5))
 (segment (start 223.5 99.9775) (end 223.5 97.77423) (width 0.25) (layer F.Cu) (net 6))
 (segment (start 213.260771 87.535001) (end 196.755001 87.535001) (width 0.25) (layer F.Cu) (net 6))
 (segment (start 196.429999 87.209999) (end 195.58 86.36) (width 0.25) (layer F.Cu) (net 6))
 (segment (start 223.5 97.77423) (end 213.260771 87.535001) (width 0.25) (layer F.Cu) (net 6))
 (segment (start 196.755001 87.535001) (end 196.429999 87.209999) (width 0.25) (layer F.Cu) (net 6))
 (segment (start 221 99.24) (end 221 99.9775) (width 0.25) (layer F.Cu) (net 11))
 (segment (start 210.82 93.98) (end 216.52372 93.98) (width 0.25) (layer F.Cu) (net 11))
 (segment (start 216.52372 93.98) (end 221 98.45628) (width 0.25) (layer F.Cu) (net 11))
 (segment (start 221 98.45628) (end 221 99.24) (width 0.25) (layer F.Cu) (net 11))
 (segment (start 210.82 96.52) (end 217.7909 96.52) (width 0.25) (layer F.Cu) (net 10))
 (segment (start 217.7909 96.52) (end 220 98.7291) (width 0.25) (layer F.Cu) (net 10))
 (segment (start 220 98.7291) (end 220 99.24) (width 0.25) (layer F.Cu) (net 10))
 (segment (start 220 99.24) (end 220 99.9775) (width 0.25) (layer F.Cu) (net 10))
 (segment (start 223 99.24) (end 223 99.9775) (width 0.25) (layer F.Cu) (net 16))
 (segment (start 223 97.91064) (end 223 99.24) (width 0.25) (layer F.Cu) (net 16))
 (segment (start 210.82 88.9) (end 213.98936 88.9) (width 0.25) (layer F.Cu) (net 16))
 (segment (start 213.98936 88.9) (end 223 97.91064) (width 0.25) (layer F.Cu) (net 16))
 (segment (start 220.5 98.59269) (end 220.5 99.24) (width 0.25) (layer F.Cu) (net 3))
 (segment (start 217.252309 95.344999) (end 220.5 98.59269) (width 0.25) (layer F.Cu) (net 3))
 (segment (start 196.944999 95.344999) (end 217.252309 95.344999) (width 0.25) (layer F.Cu) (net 3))
 (segment (start 220.5 99.24) (end 220.5 99.9775) (width 0.25) (layer F.Cu) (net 3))
 (segment (start 195.58 93.98) (end 196.944999 95.344999) (width 0.25) (layer F.Cu) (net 3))
 (segment (start 219.35 99.8275) (end 219.5 99.9775) (width 0.25) (layer F.Cu) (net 1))
 (segment (start 196.755001 97.695001) (end 217.217501 97.695001) (width 0.25) (layer F.Cu) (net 1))
 (segment (start 217.217501 97.695001) (end 219.35 99.8275) (width 0.25) (layer F.Cu) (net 1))
 (segment (start 195.58 96.52) (end 196.755001 97.695001) (width 0.25) (layer F.Cu) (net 1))
 (segment (start 218.0875 103.39) (end 218.0875 103.89) (width 0.25) (layer F.Cu) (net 2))
 (segment (start 218.0875 104.39) (end 218.0875 104.89) (width 0.25) (layer F.Cu) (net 2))
 (segment (start 217.35 103.39) (end 218.0875 103.39) (width 0.25) (layer F.Cu) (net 2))
 (segment (start 217.055 103.39) (end 217.35 103.39) (width 0.25) (layer F.Cu) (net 2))
 (segment (start 212.725 99.06) (end 217.055 103.39) (width 0.25) (layer F.Cu) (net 2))
 (segment (start 210.82 99.06) (end 212.725 99.06) (width 0.25) (layer F.Cu) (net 2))
 (segment (start 217.42 104.39) (end 218.0875 104.39) (width 0.25) (layer F.Cu) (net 2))
 (segment (start 196.85 100.33) (end 213.36 100.33) (width 0.25) (layer F.Cu) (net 2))
 (segment (start 213.36 100.33) (end 217.42 104.39) (width 0.25) (layer F.Cu) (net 2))
 (segment (start 195.58 99.06) (end 196.85 100.33) (width 0.25) (layer F.Cu) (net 2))
 (segment (start 223.5 119.4) (end 223.5 108.3025) (width 0.25) (layer F.Cu) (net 29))
 (segment (start 210.82 132.08) (end 223.5 119.4) (width 0.25) (layer F.Cu) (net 29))
 (segment (start 224 109.04) (end 224 108.3025) (width 0.25) (layer F.Cu) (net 20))
 (segment (start 224 120.639002) (end 224 109.04) (width 0.25) (layer F.Cu) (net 20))
 (segment (start 211.384001 133.255001) (end 224 120.639002) (width 0.25) (layer F.Cu) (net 20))
 (segment (start 196.755001 133.255001) (end 211.384001 133.255001) (width 0.25) (layer F.Cu) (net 20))
 (segment (start 195.58 132.08) (end 196.755001 133.255001) (width 0.25) (layer F.Cu) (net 20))
 (segment (start 195.58 84.92) (end 195.75 85.09) (width 0.25) (layer F.Cu) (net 9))
 (segment (start 195.58 83.82) (end 195.58 84.92) (width 0.25) (layer F.Cu) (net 9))
 (segment (start 224.5 99.24) (end 224.5 99.9775) (width 0.25) (layer F.Cu) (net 9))
 (segment (start 224.5 97.50141) (end 224.5 99.24) (width 0.25) (layer F.Cu) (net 9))
 (segment (start 212.08859 85.09) (end 224.5 97.50141) (width 0.25) (layer F.Cu) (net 9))
 (segment (start 195.75 85.09) (end 212.08859 85.09) (width 0.25) (layer F.Cu) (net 9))
 (segment (start 210.82 83.82) (end 211.455 83.82) (width 0.25) (layer F.Cu) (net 17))
 (segment (start 225 99.24) (end 225 99.9775) (width 0.25) (layer F.Cu) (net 17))
 (segment (start 211.455 83.82) (end 225 97.365) (width 0.25) (layer F.Cu) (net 17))
 (segment (start 225 97.365) (end 225 99.24) (width 0.25) (layer F.Cu) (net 17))
 (segment (start 224 99.24) (end 224 99.9775) (width 0.25) (layer F.Cu) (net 14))
 (segment (start 212.72218 86.36) (end 224 97.63782) (width 0.25) (layer F.Cu) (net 14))
 (segment (start 224 97.63782) (end 224 99.24) (width 0.25) (layer F.Cu) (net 14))
 (segment (start 210.82 86.36) (end 212.72218 86.36) (width 0.25) (layer F.Cu) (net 14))
 (segment (start 220 109.04) (end 220 108.3025) (width 0.25) (layer F.Cu) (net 4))
 (segment (start 220 109.105702) (end 220 109.04) (width 0.25) (layer F.Cu) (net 4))
 (segment (start 219.740692 109.36501) (end 220 109.105702) (width 0.25) (layer F.Cu) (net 4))
 (segment (start 200.80501 109.36501) (end 219.740692 109.36501) (width 0.25) (layer F.Cu) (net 4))
 (segment (start 195.58 104.14) (end 200.80501 109.36501) (width 0.25) (layer F.Cu) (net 4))
 (segment (start 195.58 120.82) (end 205.275 111.125) (width 0.25) (layer F.Cu) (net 26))
 (segment (start 195.58 121.92) (end 195.58 120.82) (width 0.25) (layer F.Cu) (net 26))
 (segment (start 220.5 109.04) (end 220.5 108.3025) (width 0.25) (layer F.Cu) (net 26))
 (segment (start 220.5 109.242112) (end 220.5 109.04) (width 0.25) (layer F.Cu) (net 26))
 (segment (start 218.617112 111.125) (end 220.5 109.242112) (width 0.25) (layer F.Cu) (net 26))
 (segment (start 205.275 111.125) (end 218.617112 111.125) (width 0.25) (layer F.Cu) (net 26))
 (segment (start 214.9825 108.3025) (end 219.5 108.3025) (width 0.25) (layer F.Cu) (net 12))
 (segment (start 210.82 104.14) (end 214.9825 108.3025) (width 0.25) (layer F.Cu) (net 12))
 (segment (start 221.5 116.32) (end 210.82 127) (width 0.25) (layer F.Cu) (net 34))
 (segment (start 221.5 108.3025) (end 221.5 116.32) (width 0.25) (layer F.Cu) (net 34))
 (segment (start 195.58 101.6) (end 196.755001 102.775001) (width 0.25) (layer F.Cu) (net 7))
 (segment (start 211.358591 102.775001) (end 215.47359 106.89) (width 0.25) (layer F.Cu) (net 7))
 (segment (start 196.755001 102.775001) (end 211.358591 102.775001) (width 0.25) (layer F.Cu) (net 7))
 (segment (start 215.47359 106.89) (end 217.35 106.89) (width 0.25) (layer F.Cu) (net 7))
 (segment (start 217.35 106.89) (end 218.0875 106.89) (width 0.25) (layer F.Cu) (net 7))
 (segment (start 195.58 124.46) (end 198.755 121.285) (width 0.25) (layer F.Cu) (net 23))
 (segment (start 198.755 121.285) (end 198.755 118.745) (width 0.25) (layer F.Cu) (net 23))
 (segment (start 221 109.04) (end 221 108.3025) (width 0.25) (layer F.Cu) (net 23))
 (segment (start 221 110.105702) (end 221 109.04) (width 0.25) (layer F.Cu) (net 23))
 (segment (start 219.530692 111.57501) (end 221 110.105702) (width 0.25) (layer F.Cu) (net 23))
 (segment (start 205.92499 111.57501) (end 219.530692 111.57501) (width 0.25) (layer F.Cu) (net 23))
 (segment (start 198.755 118.745) (end 205.92499 111.57501) (width 0.25) (layer F.Cu) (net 23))
 (segment (start 217.35 106.39) (end 218.0875 106.39) (width 0.25) (layer F.Cu) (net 15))
 (segment (start 210.82 101.6) (end 215.61 106.39) (width 0.25) (layer F.Cu) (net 15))
 (segment (start 215.61 106.39) (end 217.35 106.39) (width 0.25) (layer F.Cu) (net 15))
 (segment (start 223 109.04) (end 223 108.3025) (width 0.25) (layer F.Cu) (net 22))
 (segment (start 223 119.099002) (end 223 109.04) (width 0.25) (layer F.Cu) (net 22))
 (segment (start 211.384001 130.715001) (end 223 119.099002) (width 0.25) (layer F.Cu) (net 22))
 (segment (start 196.755001 130.715001) (end 211.384001 130.715001) (width 0.25) (layer F.Cu) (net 22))
 (segment (start 195.58 129.54) (end 196.755001 130.715001) (width 0.25) (layer F.Cu) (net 22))
 (segment (start 222.5 117.86) (end 222.5 108.3025) (width 0.25) (layer F.Cu) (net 31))
 (segment (start 210.82 129.54) (end 222.5 117.86) (width 0.25) (layer F.Cu) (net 31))
 (segment (start 196.755001 128.175001) (end 196.429999 127.849999) (width 0.25) (layer F.Cu) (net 25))
 (segment (start 196.429999 127.849999) (end 195.58 127) (width 0.25) (layer F.Cu) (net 25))
 (segment (start 211.384001 128.175001) (end 196.755001 128.175001) (width 0.25) (layer F.Cu) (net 25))
 (segment (start 222 117.559002) (end 211.384001 128.175001) (width 0.25) (layer F.Cu) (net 25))
 (segment (start 222 108.3025) (end 222 117.559002) (width 0.25) (layer F.Cu) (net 25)))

